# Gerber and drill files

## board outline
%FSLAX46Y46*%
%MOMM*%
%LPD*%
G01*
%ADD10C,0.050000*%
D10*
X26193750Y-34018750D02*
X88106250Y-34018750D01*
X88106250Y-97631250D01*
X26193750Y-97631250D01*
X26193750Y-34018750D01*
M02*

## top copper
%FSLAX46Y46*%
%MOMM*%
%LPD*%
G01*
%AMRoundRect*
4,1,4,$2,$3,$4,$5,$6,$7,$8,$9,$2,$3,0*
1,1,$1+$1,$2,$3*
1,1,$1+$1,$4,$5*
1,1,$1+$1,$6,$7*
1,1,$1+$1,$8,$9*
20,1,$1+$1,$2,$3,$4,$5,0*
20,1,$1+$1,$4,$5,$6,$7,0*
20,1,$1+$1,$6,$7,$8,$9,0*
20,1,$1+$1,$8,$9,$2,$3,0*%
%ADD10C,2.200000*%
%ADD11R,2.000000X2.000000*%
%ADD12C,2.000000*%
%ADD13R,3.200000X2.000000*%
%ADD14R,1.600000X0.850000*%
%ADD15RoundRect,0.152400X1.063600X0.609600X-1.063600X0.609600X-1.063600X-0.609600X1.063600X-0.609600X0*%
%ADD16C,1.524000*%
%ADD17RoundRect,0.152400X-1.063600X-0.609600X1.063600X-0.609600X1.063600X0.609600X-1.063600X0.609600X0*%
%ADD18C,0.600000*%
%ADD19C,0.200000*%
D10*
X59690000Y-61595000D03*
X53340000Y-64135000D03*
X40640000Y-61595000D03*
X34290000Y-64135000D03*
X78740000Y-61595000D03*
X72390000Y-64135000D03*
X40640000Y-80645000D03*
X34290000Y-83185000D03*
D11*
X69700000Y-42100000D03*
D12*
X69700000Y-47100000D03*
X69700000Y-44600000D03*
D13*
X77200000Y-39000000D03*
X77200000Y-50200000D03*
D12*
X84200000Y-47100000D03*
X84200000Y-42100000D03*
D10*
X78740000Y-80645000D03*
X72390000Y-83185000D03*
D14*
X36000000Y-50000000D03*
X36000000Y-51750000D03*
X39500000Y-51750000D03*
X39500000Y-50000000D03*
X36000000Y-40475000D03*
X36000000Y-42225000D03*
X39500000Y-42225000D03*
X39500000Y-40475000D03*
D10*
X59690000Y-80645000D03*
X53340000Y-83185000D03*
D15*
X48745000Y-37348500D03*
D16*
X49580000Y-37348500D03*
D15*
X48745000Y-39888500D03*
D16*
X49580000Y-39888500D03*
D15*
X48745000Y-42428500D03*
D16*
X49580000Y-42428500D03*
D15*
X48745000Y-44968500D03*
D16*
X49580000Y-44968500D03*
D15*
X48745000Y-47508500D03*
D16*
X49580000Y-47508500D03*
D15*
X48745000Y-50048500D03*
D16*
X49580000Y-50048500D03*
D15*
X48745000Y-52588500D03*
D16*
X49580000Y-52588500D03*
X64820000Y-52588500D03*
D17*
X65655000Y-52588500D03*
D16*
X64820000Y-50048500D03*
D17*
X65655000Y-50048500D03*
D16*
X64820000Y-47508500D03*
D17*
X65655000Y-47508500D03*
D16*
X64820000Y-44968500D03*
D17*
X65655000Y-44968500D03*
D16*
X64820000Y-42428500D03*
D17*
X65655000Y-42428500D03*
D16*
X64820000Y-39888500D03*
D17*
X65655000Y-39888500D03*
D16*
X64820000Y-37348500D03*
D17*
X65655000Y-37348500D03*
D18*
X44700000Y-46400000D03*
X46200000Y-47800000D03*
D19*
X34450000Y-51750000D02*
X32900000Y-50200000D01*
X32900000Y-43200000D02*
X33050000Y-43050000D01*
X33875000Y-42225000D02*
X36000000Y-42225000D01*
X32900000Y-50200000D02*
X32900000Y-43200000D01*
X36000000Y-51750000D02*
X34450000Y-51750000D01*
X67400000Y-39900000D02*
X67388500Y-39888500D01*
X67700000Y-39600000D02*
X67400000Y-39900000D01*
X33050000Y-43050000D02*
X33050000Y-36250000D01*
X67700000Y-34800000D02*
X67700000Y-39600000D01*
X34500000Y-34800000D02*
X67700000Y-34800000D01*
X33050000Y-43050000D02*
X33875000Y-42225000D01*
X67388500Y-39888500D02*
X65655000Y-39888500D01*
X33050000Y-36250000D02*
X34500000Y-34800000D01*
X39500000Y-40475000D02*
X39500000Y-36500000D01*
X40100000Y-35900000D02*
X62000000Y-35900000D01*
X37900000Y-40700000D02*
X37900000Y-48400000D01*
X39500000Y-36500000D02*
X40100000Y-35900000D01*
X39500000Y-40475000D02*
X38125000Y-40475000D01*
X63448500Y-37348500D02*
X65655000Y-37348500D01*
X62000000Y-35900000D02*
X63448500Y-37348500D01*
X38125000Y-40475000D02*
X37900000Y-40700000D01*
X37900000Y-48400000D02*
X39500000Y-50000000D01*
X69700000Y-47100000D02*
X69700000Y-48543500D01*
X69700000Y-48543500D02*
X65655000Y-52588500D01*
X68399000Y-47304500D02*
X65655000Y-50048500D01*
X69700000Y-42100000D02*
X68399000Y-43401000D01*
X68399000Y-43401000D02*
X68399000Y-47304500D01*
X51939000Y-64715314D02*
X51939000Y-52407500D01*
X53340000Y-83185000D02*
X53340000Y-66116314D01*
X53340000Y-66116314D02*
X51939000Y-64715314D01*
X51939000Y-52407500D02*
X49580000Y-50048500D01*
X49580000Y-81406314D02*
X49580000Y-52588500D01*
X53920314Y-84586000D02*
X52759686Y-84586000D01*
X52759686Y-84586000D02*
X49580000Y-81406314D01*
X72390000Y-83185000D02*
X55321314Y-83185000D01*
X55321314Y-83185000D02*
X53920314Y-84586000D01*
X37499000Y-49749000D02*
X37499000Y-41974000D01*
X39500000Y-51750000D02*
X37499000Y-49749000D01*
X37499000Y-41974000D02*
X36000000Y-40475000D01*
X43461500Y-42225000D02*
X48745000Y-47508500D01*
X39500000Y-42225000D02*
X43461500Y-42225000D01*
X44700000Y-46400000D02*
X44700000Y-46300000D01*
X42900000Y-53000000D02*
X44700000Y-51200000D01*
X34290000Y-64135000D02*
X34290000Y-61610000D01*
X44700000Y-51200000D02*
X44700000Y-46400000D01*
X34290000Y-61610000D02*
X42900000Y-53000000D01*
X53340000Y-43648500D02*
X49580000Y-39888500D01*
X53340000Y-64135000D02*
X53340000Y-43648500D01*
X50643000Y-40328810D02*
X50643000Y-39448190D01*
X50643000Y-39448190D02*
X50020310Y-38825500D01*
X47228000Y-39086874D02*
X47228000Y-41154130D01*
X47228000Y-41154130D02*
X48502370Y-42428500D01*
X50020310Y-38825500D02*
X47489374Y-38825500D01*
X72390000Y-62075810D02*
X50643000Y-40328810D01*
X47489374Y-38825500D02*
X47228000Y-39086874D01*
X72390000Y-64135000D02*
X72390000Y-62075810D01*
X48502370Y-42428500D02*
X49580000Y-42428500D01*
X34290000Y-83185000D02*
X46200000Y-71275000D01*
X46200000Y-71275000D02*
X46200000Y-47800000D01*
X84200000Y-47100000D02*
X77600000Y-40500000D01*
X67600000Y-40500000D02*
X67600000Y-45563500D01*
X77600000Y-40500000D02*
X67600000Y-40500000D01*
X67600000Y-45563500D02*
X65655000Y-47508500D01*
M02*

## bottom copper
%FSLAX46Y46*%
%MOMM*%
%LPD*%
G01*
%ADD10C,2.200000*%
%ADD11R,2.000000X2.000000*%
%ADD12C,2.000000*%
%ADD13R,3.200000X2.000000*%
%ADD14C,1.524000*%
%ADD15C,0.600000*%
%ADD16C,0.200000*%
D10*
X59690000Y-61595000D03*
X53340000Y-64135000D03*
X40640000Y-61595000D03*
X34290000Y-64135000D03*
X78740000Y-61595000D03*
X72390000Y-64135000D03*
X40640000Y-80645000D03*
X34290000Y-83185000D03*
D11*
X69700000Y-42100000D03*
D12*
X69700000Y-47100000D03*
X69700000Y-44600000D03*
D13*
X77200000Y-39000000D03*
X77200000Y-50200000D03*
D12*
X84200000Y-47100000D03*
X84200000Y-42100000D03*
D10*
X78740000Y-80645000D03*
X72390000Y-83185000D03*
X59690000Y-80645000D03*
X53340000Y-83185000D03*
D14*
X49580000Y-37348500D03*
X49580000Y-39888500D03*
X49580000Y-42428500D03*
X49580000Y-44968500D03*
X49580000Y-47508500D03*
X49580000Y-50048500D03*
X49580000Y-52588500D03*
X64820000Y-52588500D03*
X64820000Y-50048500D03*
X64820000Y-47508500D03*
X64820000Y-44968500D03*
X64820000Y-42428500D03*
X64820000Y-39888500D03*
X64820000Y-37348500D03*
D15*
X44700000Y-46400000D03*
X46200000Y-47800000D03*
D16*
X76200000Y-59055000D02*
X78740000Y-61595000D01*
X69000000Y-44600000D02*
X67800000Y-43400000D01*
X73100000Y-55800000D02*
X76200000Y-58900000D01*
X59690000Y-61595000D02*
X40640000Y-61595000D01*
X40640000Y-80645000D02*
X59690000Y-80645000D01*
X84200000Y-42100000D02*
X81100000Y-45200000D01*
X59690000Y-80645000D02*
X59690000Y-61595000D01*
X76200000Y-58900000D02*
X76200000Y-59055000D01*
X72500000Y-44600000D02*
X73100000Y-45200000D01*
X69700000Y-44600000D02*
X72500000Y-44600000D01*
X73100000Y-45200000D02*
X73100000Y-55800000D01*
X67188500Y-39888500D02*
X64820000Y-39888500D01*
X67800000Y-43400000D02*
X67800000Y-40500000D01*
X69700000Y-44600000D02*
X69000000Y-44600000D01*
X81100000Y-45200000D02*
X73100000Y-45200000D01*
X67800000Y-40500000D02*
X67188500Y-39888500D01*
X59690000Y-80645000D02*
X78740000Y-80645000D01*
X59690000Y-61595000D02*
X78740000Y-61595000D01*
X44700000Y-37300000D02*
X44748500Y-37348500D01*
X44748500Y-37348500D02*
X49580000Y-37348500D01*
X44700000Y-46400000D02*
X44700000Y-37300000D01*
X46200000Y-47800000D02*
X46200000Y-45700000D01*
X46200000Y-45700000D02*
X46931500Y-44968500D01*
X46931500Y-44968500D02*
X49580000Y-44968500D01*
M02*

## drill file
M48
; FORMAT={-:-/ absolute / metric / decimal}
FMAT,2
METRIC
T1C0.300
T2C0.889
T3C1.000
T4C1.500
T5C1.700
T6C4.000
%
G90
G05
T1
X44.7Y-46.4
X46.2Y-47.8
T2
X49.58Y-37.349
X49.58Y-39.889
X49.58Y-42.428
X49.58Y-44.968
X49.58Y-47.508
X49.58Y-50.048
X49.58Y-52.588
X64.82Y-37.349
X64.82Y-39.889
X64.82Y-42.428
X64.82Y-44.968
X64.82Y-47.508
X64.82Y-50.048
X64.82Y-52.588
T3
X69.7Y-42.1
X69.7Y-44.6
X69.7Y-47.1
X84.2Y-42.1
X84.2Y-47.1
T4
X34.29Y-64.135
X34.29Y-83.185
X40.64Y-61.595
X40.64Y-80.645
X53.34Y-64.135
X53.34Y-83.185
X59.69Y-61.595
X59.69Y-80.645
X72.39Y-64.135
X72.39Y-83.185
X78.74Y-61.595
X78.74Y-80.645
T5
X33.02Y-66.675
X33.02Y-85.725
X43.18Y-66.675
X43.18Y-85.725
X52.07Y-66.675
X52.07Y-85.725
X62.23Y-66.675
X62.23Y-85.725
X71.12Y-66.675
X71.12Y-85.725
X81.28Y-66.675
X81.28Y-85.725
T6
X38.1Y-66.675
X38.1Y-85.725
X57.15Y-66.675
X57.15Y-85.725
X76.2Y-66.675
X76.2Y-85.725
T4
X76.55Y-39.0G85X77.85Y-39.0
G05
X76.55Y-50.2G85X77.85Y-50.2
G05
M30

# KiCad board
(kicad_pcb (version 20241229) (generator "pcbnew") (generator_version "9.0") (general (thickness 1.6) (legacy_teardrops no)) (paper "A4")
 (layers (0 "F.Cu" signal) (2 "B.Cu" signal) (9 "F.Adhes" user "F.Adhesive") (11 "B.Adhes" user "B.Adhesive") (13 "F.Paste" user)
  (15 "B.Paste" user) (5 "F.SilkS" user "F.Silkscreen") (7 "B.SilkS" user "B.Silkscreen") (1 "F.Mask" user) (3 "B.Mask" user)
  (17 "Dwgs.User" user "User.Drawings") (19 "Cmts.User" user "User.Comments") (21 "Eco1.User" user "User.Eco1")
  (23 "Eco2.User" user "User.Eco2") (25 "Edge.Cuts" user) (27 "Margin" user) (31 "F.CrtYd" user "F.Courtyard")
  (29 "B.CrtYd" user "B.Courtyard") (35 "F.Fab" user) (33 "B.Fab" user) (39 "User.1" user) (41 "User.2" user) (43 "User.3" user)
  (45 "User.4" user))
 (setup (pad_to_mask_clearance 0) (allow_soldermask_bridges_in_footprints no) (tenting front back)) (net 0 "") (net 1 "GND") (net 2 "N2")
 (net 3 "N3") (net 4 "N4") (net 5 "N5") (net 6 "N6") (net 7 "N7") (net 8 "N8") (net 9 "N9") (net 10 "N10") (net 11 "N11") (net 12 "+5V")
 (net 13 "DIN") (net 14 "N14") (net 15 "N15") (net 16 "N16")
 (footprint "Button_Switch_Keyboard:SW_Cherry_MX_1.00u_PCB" (layer "F.Cu") (at 59.69 61.595)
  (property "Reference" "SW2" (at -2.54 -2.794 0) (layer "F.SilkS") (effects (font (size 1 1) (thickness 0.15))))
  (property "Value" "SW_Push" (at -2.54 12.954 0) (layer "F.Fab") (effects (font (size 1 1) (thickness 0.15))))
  (pad "" np_thru_hole circle (at -7.62 5.08) (size 1.7 1.7) (drill 1.7) (layers "*.Cu" "*.Mask"))
  (pad "" np_thru_hole circle (at -2.54 5.08) (size 4 4) (drill 4) (layers "*.Cu" "*.Mask"))
  (pad "" np_thru_hole circle (at 2.54 5.08) (size 1.7 1.7) (drill 1.7) (layers "*.Cu" "*.Mask"))
  (pad "1" thru_hole circle (at 0 0) (size 2.2 2.2) (drill 1.5) (layers "*.Cu" "*.Mask") (remove_unused_layers no) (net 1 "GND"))
  (pad "2" thru_hole circle (at -6.35 2.54) (size 2.2 2.2) (drill 1.5) (layers "*.Cu" "*.Mask") (remove_unused_layers no) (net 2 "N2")))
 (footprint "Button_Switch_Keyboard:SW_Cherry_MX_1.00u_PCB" (layer "F.Cu") (at 40.64 61.595)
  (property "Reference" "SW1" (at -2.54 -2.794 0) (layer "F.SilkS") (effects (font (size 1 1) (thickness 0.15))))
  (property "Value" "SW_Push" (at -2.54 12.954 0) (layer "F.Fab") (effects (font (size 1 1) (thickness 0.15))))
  (pad "" np_thru_hole circle (at -7.62 5.08) (size 1.7 1.7) (drill 1.7) (layers "*.Cu" "*.Mask"))
  (pad "" np_thru_hole circle (at -2.54 5.08) (size 4 4) (drill 4) (layers "*.Cu" "*.Mask"))
  (pad "" np_thru_hole circle (at 2.54 5.08) (size 1.7 1.7) (drill 1.7) (layers "*.Cu" "*.Mask"))
  (pad "1" thru_hole circle (at 0 0) (size 2.2 2.2) (drill 1.5) (layers "*.Cu" "*.Mask") (remove_unused_layers no) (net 1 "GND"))
  (pad "2" thru_hole circle (at -6.35 2.54) (size 2.2 2.2) (drill 1.5) (layers "*.Cu" "*.Mask") (remove_unused_layers no) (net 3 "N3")))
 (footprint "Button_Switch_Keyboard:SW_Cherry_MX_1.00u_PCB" (layer "F.Cu") (at 78.74 61.595)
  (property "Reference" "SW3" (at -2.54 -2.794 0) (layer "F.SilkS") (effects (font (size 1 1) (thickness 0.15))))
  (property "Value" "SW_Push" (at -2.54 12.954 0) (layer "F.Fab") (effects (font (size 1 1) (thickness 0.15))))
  (pad "" np_thru_hole circle (at -7.62 5.08) (size 1.7 1.7) (drill 1.7) (layers "*.Cu" "*.Mask"))
  (pad "" np_thru_hole circle (at -2.54 5.08) (size 4 4) (drill 4) (layers "*.Cu" "*.Mask"))
  (pad "" np_thru_hole circle (at 2.54 5.08) (size 1.7 1.7) (drill 1.7) (layers "*.Cu" "*.Mask"))
  (pad "1" thru_hole circle (at 0 0) (size 2.2 2.2) (drill 1.5) (layers "*.Cu" "*.Mask") (remove_unused_layers no) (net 1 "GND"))
  (pad "2" thru_hole circle (at -6.35 2.54) (size 2.2 2.2) (drill 1.5) (layers "*.Cu" "*.Mask") (remove_unused_layers no) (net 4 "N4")))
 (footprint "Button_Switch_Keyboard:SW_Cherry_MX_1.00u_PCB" (layer "F.Cu") (at 40.64 80.645)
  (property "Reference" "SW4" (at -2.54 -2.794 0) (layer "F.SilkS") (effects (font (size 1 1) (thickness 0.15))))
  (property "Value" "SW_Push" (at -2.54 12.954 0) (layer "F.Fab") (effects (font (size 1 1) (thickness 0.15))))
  (pad "" np_thru_hole circle (at -7.62 5.08) (size 1.7 1.7) (drill 1.7) (layers "*.Cu" "*.Mask"))
  (pad "" np_thru_hole circle (at -2.54 5.08) (size 4 4) (drill 4) (layers "*.Cu" "*.Mask"))
  (pad "" np_thru_hole circle (at 2.54 5.08) (size 1.7 1.7) (drill 1.7) (layers "*.Cu" "*.Mask"))
  (pad "1" thru_hole circle (at 0 0) (size 2.2 2.2) (drill 1.5) (layers "*.Cu" "*.Mask") (remove_unused_layers no) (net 1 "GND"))
  (pad "2" thru_hole circle (at -6.35 2.54) (size 2.2 2.2) (drill 1.5) (layers "*.Cu" "*.Mask") (remove_unused_layers no) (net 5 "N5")))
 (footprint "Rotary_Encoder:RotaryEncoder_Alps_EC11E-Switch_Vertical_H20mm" (layer "F.Cu") (at 69.7 42.1)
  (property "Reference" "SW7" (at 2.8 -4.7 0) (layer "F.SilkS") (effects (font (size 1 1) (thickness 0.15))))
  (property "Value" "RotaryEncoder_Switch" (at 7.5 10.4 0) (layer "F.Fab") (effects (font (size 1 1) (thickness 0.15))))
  (pad "A" thru_hole rect (at 0 0) (size 2 2) (drill 1) (layers "*.Cu" "*.Mask") (remove_unused_layers no) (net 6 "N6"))
  (pad "B" thru_hole circle (at 0 5) (size 2 2) (drill 1) (layers "*.Cu" "*.Mask") (remove_unused_layers no) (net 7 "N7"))
  (pad "C" thru_hole circle (at 0 2.5) (size 2 2) (drill 1) (layers "*.Cu" "*.Mask") (remove_unused_layers no) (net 1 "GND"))
  (pad "MP" thru_hole rect (at 7.5 -3.1) (size 3.2 2) (drill oval 2.8 1.5) (layers "*.Cu" "*.Mask") (remove_unused_layers no))
  (pad "MP" thru_hole rect (at 7.5 8.1) (size 3.2 2) (drill oval 2.8 1.5) (layers "*.Cu" "*.Mask") (remove_unused_layers no))
  (pad "S1" thru_hole circle (at 14.5 5) (size 2 2) (drill 1) (layers "*.Cu" "*.Mask") (remove_unused_layers no) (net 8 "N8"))
  (pad "S2" thru_hole circle (at 14.5 0) (size 2 2) (drill 1) (layers "*.Cu" "*.Mask") (remove_unused_layers no) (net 1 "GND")))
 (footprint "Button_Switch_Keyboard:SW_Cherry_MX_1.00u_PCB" (layer "F.Cu") (at 78.74 80.645)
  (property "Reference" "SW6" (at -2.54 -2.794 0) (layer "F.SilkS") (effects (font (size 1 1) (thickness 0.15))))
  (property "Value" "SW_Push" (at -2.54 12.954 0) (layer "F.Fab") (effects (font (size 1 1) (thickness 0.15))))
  (pad "" np_thru_hole circle (at -7.62 5.08) (size 1.7 1.7) (drill 1.7) (layers "*.Cu" "*.Mask"))
  (pad "" np_thru_hole circle (at -2.54 5.08) (size 4 4) (drill 4) (layers "*.Cu" "*.Mask"))
  (pad "" np_thru_hole circle (at 2.54 5.08) (size 1.7 1.7) (drill 1.7) (layers "*.Cu" "*.Mask"))
  (pad "1" thru_hole circle (at 0 0) (size 2.2 2.2) (drill 1.5) (layers "*.Cu" "*.Mask") (remove_unused_layers no) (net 1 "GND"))
  (pad "2" thru_hole circle (at -6.35 2.54) (size 2.2 2.2) (drill 1.5) (layers "*.Cu" "*.Mask") (remove_unused_layers no) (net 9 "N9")))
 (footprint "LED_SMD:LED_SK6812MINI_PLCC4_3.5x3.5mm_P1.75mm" (layer "F.Cu") (at 37.75 50.875)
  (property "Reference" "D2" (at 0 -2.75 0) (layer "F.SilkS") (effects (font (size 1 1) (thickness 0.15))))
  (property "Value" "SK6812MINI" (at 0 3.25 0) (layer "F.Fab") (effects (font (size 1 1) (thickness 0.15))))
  (pad "1" smd rect (at -1.75 -0.875) (size 1.6 0.85) (layers "F.Cu" "F.Mask" "F.Paste") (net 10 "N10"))
  (pad "2" smd rect (at -1.75 0.875) (size 1.6 0.85) (layers "F.Cu" "F.Mask" "F.Paste") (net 1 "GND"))
  (pad "3" smd rect (at 1.75 0.875) (size 1.6 0.85) (layers "F.Cu" "F.Mask" "F.Paste") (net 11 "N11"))
  (pad "4" smd rect (at 1.75 -0.875) (size 1.6 0.85) (layers "F.Cu" "F.Mask" "F.Paste") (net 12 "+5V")))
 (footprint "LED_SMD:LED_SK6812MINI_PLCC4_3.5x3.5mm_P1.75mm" (layer "F.Cu") (at 37.75 41.35)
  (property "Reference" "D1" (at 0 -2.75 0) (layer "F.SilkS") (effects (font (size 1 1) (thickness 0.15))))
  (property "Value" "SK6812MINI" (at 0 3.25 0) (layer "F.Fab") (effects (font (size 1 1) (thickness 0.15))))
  (pad "1" smd rect (at -1.75 -0.875) (size 1.6 0.85) (layers "F.Cu" "F.Mask" "F.Paste") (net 11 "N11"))
  (pad "2" smd rect (at -1.75 0.875) (size 1.6 0.85) (layers "F.Cu" "F.Mask" "F.Paste") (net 1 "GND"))
  (pad "3" smd rect (at 1.75 0.875) (size 1.6 0.85) (layers "F.Cu" "F.Mask" "F.Paste") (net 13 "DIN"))
  (pad "4" smd rect (at 1.75 -0.875) (size 1.6 0.85) (layers "F.Cu" "F.Mask" "F.Paste") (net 12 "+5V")))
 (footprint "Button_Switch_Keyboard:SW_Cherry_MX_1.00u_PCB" (layer "F.Cu") (at 59.69 80.645)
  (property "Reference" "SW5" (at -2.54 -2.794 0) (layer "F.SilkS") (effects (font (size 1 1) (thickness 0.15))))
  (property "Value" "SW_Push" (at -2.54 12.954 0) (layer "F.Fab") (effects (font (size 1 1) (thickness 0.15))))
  (pad "" np_thru_hole circle (at -7.62 5.08) (size 1.7 1.7) (drill 1.7) (layers "*.Cu" "*.Mask"))
  (pad "" np_thru_hole circle (at -2.54 5.08) (size 4 4) (drill 4) (layers "*.Cu" "*.Mask"))
  (pad "" np_thru_hole circle (at 2.54 5.08) (size 1.7 1.7) (drill 1.7) (layers "*.Cu" "*.Mask"))
  (pad "1" thru_hole circle (at 0 0) (size 2.2 2.2) (drill 1.5) (layers "*.Cu" "*.Mask") (remove_unused_layers no) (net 1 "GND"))
  (pad "2" thru_hole circle (at -6.35 2.54) (size 2.2 2.2) (drill 1.5) (layers "*.Cu" "*.Mask") (remove_unused_layers no) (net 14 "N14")))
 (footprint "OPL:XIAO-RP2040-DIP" (layer "F.Cu") (at 57.2 44.9685)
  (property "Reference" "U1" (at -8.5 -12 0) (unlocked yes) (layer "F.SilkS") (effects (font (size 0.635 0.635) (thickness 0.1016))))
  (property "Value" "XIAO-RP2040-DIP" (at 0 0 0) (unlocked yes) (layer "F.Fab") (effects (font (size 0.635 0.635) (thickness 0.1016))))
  (pad "1" smd roundrect (at -8.455 -7.62 180) (size 2.432 1.524) (layers "F.Cu" "F.Mask") (roundrect_rratio 0.1) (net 3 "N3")
   (thermal_bridge_angle 45))
  (pad "1" thru_hole circle (at -7.62 -7.62 180) (size 1.524 1.524) (drill 0.889) (layers "*.Cu" "*.Mask") (remove_unused_layers no)
   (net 3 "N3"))
  (pad "2" smd roundrect (at -8.455 -5.08 180) (size 2.432 1.524) (layers "F.Cu" "F.Mask") (roundrect_rratio 0.1) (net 2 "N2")
   (thermal_bridge_angle 45))
  (pad "2" thru_hole circle (at -7.62 -5.08 180) (size 1.524 1.524) (drill 0.889) (layers "*.Cu" "*.Mask") (remove_unused_layers no)
   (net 2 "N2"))
  (pad "3" smd roundrect (at -8.455 -2.54 180) (size 2.432 1.524) (layers "F.Cu" "F.Mask") (roundrect_rratio 0.1) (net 4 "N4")
   (thermal_bridge_angle 45))
  (pad "3" thru_hole circle (at -7.62 -2.54 180) (size 1.524 1.524) (drill 0.889) (layers "*.Cu" "*.Mask") (remove_unused_layers no)
   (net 4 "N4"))
  (pad "4" smd roundrect (at -8.455 0 180) (size 2.432 1.524) (layers "F.Cu" "F.Mask") (roundrect_rratio 0.1) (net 5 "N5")
   (thermal_bridge_angle 45))
  (pad "4" thru_hole circle (at -7.62 0 180) (size 1.524 1.524) (drill 0.889) (layers "*.Cu" "*.Mask") (remove_unused_layers no)
   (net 5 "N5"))
  (pad "5" smd roundrect (at -8.455 2.54 180) (size 2.432 1.524) (layers "F.Cu" "F.Mask") (roundrect_rratio 0.1) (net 13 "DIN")
   (thermal_bridge_angle 45))
  (pad "5" thru_hole circle (at -7.62 2.54 180) (size 1.524 1.524) (drill 0.889) (layers "*.Cu" "*.Mask") (remove_unused_layers no)
   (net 13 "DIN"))
  (pad "6" smd roundrect (at -8.455 5.08 180) (size 2.432 1.524) (layers "F.Cu" "F.Mask") (roundrect_rratio 0.1) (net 14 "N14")
   (thermal_bridge_angle 45))
  (pad "6" thru_hole circle (at -7.62 5.08 180) (size 1.524 1.524) (drill 0.889) (layers "*.Cu" "*.Mask") (remove_unused_layers no)
   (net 14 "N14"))
  (pad "7" smd roundrect (at -8.455 7.62 180) (size 2.432 1.524) (layers "F.Cu" "F.Mask") (roundrect_rratio 0.1) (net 9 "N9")
   (thermal_bridge_angle 45))
  (pad "7" thru_hole circle (at -7.62 7.62 180) (size 1.524 1.524) (drill 0.889) (layers "*.Cu" "*.Mask") (remove_unused_layers no)
   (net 9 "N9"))
  (pad "8" thru_hole circle (at 7.62 7.62) (size 1.524 1.524) (drill 0.889) (layers "*.Cu" "*.Mask") (remove_unused_layers no) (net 7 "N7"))
  (pad "8" smd roundrect (at 8.455 7.62) (size 2.432 1.524) (layers "F.Cu" "F.Mask") (roundrect_rratio 0.1) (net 7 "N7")
   (thermal_bridge_angle 45))
  (pad "9" thru_hole circle (at 7.62 5.08) (size 1.524 1.524) (drill 0.889) (layers "*.Cu" "*.Mask") (remove_unused_layers no) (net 6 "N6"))
  (pad "9" smd roundrect (at 8.455 5.08) (size 2.432 1.524) (layers "F.Cu" "F.Mask") (roundrect_rratio 0.1) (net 6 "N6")
   (thermal_bridge_angle 45))
  (pad "10" thru_hole circle (at 7.62 2.54) (size 1.524 1.524) (drill 0.889) (layers "*.Cu" "*.Mask") (remove_unused_layers no) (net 8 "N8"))
  (pad "10" smd roundrect (at 8.455 2.54) (size 2.432 1.524) (layers "F.Cu" "F.Mask") (roundrect_rratio 0.1) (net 8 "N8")
   (thermal_bridge_angle 45))
  (pad "11" thru_hole circle (at 7.62 0) (size 1.524 1.524) (drill 0.889) (layers "*.Cu" "*.Mask") (remove_unused_layers no) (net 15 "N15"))
  (pad "11" smd roundrect (at 8.455 0) (size 2.432 1.524) (layers "F.Cu" "F.Mask") (roundrect_rratio 0.1) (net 15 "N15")
   (thermal_bridge_angle 45))
  (pad "12" thru_hole circle (at 7.62 -2.54) (size 1.524 1.524) (drill 0.889) (layers "*.Cu" "*.Mask") (remove_unused_layers no)
   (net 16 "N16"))
  (pad "12" smd roundrect (at 8.455 -2.54) (size 2.432 1.524) (layers "F.Cu" "F.Mask") (roundrect_rratio 0.1) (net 16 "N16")
   (thermal_bridge_angle 45))
  (pad "13" thru_hole circle (at 7.62 -5.08) (size 1.524 1.524) (drill 0.889) (layers "*.Cu" "*.Mask") (remove_unused_layers no)
   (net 1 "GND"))
  (pad "13" smd roundrect (at 8.455 -5.08) (size 2.432 1.524) (layers "F.Cu" "F.Mask") (roundrect_rratio 0.1) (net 1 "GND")
   (thermal_bridge_angle 45))
  (pad "14" thru_hole circle (at 7.62 -7.62) (size 1.524 1.524) (drill 0.889) (layers "*.Cu" "*.Mask") (remove_unused_layers no)
   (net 12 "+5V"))
  (pad "14" smd roundrect (at 8.455 -7.62) (size 2.432 1.524) (layers "F.Cu" "F.Mask") (roundrect_rratio 0.1) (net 12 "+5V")
   (thermal_bridge_angle 45)))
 (gr_rect (start 26.19375 34.01875) (end 88.10625 97.63125) (stroke (width 0.05) (type default)) (fill no) (layer "Edge.Cuts"))
 (segment (start 34.45 51.75) (end 32.9 50.2) (width 0.2) (layer "F.Cu") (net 1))
 (segment (start 32.9 43.2) (end 33.05 43.05) (width 0.2) (layer "F.Cu") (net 1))
 (segment (start 33.875 42.225) (end 36 42.225) (width 0.2) (layer "F.Cu") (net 1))
 (segment (start 32.9 50.2) (end 32.9 43.2) (width 0.2) (layer "F.Cu") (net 1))
 (segment (start 36 51.75) (end 34.45 51.75) (width 0.2) (layer "F.Cu") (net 1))
 (segment (start 67.4 39.9) (end 67.3885 39.8885) (width 0.2) (layer "F.Cu") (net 1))
 (segment (start 67.7 39.6) (end 67.4 39.9) (width 0.2) (layer "F.Cu") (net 1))
 (segment (start 33.05 43.05) (end 33.05 36.25) (width 0.2) (layer "F.Cu") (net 1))
 (segment (start 67.7 34.8) (end 67.7 39.6) (width 0.2) (layer "F.Cu") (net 1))
 (segment (start 34.5 34.8) (end 67.7 34.8) (width 0.2) (layer "F.Cu") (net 1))
 (segment (start 33.05 43.05) (end 33.875 42.225) (width 0.2) (layer "F.Cu") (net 1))
 (segment (start 67.3885 39.8885) (end 65.655 39.8885) (width 0.2) (layer "F.Cu") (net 1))
 (segment (start 33.05 36.25) (end 34.5 34.8) (width 0.2) (layer "F.Cu") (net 1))
 (segment (start 76.2 59.055) (end 78.74 61.595) (width 0.2) (layer "B.Cu") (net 1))
 (segment (start 69 44.6) (end 67.8 43.4) (width 0.2) (layer "B.Cu") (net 1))
 (segment (start 73.1 55.8) (end 76.2 58.9) (width 0.2) (layer "B.Cu") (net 1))
 (segment (start 59.69 61.595) (end 40.64 61.595) (width 0.2) (layer "B.Cu") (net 1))
 (segment (start 40.64 80.645) (end 59.69 80.645) (width 0.2) (layer "B.Cu") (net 1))
 (segment (start 84.2 42.1) (end 81.1 45.2) (width 0.2) (layer "B.Cu") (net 1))
 (segment (start 59.69 80.645) (end 59.69 61.595) (width 0.2) (layer "B.Cu") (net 1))
 (segment (start 76.2 58.9) (end 76.2 59.055) (width 0.2) (layer "B.Cu") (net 1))
 (segment (start 72.5 44.6) (end 73.1 45.2) (width 0.2) (layer "B.Cu") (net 1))
 (segment (start 69.7 44.6) (end 72.5 44.6) (width 0.2) (layer "B.Cu") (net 1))
 (segment (start 73.1 45.2) (end 73.1 55.8) (width 0.2) (layer "B.Cu") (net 1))
 (segment (start 67.1885 39.8885) (end 64.82 39.8885) (width 0.2) (layer "B.Cu") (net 1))
 (segment (start 67.8 43.4) (end 67.8 40.5) (width 0.2) (layer "B.Cu") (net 1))
 (segment (start 69.7 44.6) (end 69 44.6) (width 0.2) (layer "B.Cu") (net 1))
 (segment (start 81.1 45.2) (end 73.1 45.2) (width 0.2) (layer "B.Cu") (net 1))
 (segment (start 67.8 40.5) (end 67.1885 39.8885) (width 0.2) (layer "B.Cu") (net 1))
 (segment (start 59.69 80.645) (end 78.74 80.645) (width 0.2) (layer "B.Cu") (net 1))
 (segment (start 59.69 61.595) (end 78.74 61.595) (width 0.2) (layer "B.Cu") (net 1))
 (segment (start 39.5 40.475) (end 39.5 36.5) (width 0.2) (layer "F.Cu") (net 12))
 (segment (start 40.1 35.9) (end 62 35.9) (width 0.2) (layer "F.Cu") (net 12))
 (segment (start 37.9 40.7) (end 37.9 48.4) (width 0.2) (layer "F.Cu") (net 12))
 (segment (start 39.5 36.5) (end 40.1 35.9) (width 0.2) (layer "F.Cu") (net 12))
 (segment (start 39.5 40.475) (end 38.125 40.475) (width 0.2) (layer "F.Cu") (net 12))
 (segment (start 63.4485 37.3485) (end 65.655 37.3485) (width 0.2) (layer "F.Cu") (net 12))
 (segment (start 62 35.9) (end 63.4485 37.3485) (width 0.2) (layer "F.Cu") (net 12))
 (segment (start 38.125 40.475) (end 37.9 40.7) (width 0.2) (layer "F.Cu") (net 12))
 (segment (start 37.9 48.4) (end 39.5 50) (width 0.2) (layer "F.Cu") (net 12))
 (segment (start 69.7 47.1) (end 69.7 48.5435) (width 0.2) (layer "F.Cu") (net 7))
 (segment (start 69.7 48.5435) (end 65.655 52.5885) (width 0.2) (layer "F.Cu") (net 7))
 (segment (start 68.399 47.3045) (end 65.655 50.0485) (width 0.2) (layer "F.Cu") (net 6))
 (segment (start 69.7 42.1) (end 68.399 43.401) (width 0.2) (layer "F.Cu") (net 6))
 (segment (start 68.399 43.401) (end 68.399 47.3045) (width 0.2) (layer "F.Cu") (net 6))
 (segment (start 51.939 64.715314) (end 51.939 52.4075) (width 0.2) (layer "F.Cu") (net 14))
 (segment (start 53.34 83.185) (end 53.34 66.116314) (width 0.2) (layer "F.Cu") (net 14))
 (segment (start 53.34 66.116314) (end 51.939 64.715314) (width 0.2) (layer "F.Cu") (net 14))
 (segment (start 51.939 52.4075) (end 49.58 50.0485) (width 0.2) (layer "F.Cu") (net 14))
 (segment (start 49.58 81.406314) (end 49.58 52.5885) (width 0.2) (layer "F.Cu") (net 9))
 (segment (start 53.920314 84.586) (end 52.759686 84.586) (width 0.2) (layer "F.Cu") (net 9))
 (segment (start 52.759686 84.586) (end 49.58 81.406314) (width 0.2) (layer "F.Cu") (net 9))
 (segment (start 72.39 83.185) (end 55.321314 83.185) (width 0.2) (layer "F.Cu") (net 9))
 (segment (start 55.321314 83.185) (end 53.920314 84.586) (width 0.2) (layer "F.Cu") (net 9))
 (segment (start 37.499 49.749) (end 37.499 41.974) (width 0.2) (layer "F.Cu") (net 11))
 (segment (start 39.5 51.75) (end 37.499 49.749) (width 0.2) (layer "F.Cu") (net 11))
 (segment (start 37.499 41.974) (end 36 40.475) (width 0.2) (layer "F.Cu") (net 11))
 (segment (start 43.4615 42.225) (end 48.745 47.5085) (width 0.2) (layer "F.Cu") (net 13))
 (segment (start 39.5 42.225) (end 43.4615 42.225) (width 0.2) (layer "F.Cu") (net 13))
 (segment (start 44.7 46.4) (end 44.7 46.3) (width 0.2) (layer "F.Cu") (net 3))
 (segment (start 42.9 53) (end 44.7 51.2) (width 0.2) (layer "F.Cu") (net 3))
 (segment (start 34.29 64.135) (end 34.29 61.61) (width 0.2) (layer "F.Cu") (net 3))
 (segment (start 44.7 51.2) (end 44.7 46.4) (width 0.2) (layer "F.Cu") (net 3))
 (segment (start 34.29 61.61) (end 42.9 53) (width 0.2) (layer "F.Cu") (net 3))
 (via (at 44.7 46.4) (size 0.6) (drill 0.3) (layers "F.Cu" "B.Cu") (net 3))
 (segment (start 44.7 37.3) (end 44.7485 37.3485) (width 0.2) (layer "B.Cu") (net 3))
 (segment (start 44.7485 37.3485) (end 49.58 37.3485) (width 0.2) (layer "B.Cu") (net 3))
 (segment (start 44.7 46.4) (end 44.7 37.3) (width 0.2) (layer "B.Cu") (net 3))
 (segment (start 53.34 43.6485) (end 49.58 39.8885) (width 0.2) (layer "F.Cu") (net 2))
 (segment (start 53.34 64.135) (end 53.34 43.6485) (width 0.2) (layer "F.Cu") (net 2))
 (segment (start 50.643 40.32881) (end 50.643 39.44819) (width 0.2) (layer "F.Cu") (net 4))
 (segment (start 50.643 39.44819) (end 50.02031 38.8255) (width 0.2) (layer "F.Cu") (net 4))
 (segment (start 47.228 39.086874) (end 47.228 41.15413) (width 0.2) (layer "F.Cu") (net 4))
 (segment (start 47.228 41.15413) (end 48.50237 42.4285) (width 0.2) (layer "F.Cu") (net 4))
 (segment (start 50.02031 38.8255) (end 47.489374 38.8255) (width 0.2) (layer "F.Cu") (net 4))
 (segment (start 72.39 62.07581) (end 50.643 40.32881) (width 0.2) (layer "F.Cu") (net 4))
 (segment (start 47.489374 38.8255) (end 47.228 39.086874) (width 0.2) (layer "F.Cu") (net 4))
 (segment (start 72.39 64.135) (end 72.39 62.07581) (width 0.2) (layer "F.Cu") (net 4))
 (segment (start 48.50237 42.4285) (end 49.58 42.4285) (width 0.2) (layer "F.Cu") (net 4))
 (segment (start 34.29 83.185) (end 46.2 71.275) (width 0.2) (layer "F.Cu") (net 5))
 (segment (start 46.2 71.275) (end 46.2 47.8) (width 0.2) (layer "F.Cu") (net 5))
 (via (at 46.2 47.8) (size 0.6) (drill 0.3) (layers "F.Cu" "B.Cu") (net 5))
 (segment (start 46.2 47.8) (end 46.2 45.7) (width 0.2) (layer "B.Cu") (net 5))
 (segment (start 46.2 45.7) (end 46.9315 44.9685) (width 0.2) (layer "B.Cu") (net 5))
 (segment (start 46.9315 44.9685) (end 49.58 44.9685) (width 0.2) (layer "B.Cu") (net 5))
 (segment (start 84.2 47.1) (end 77.6 40.5) (width 0.2) (layer "F.Cu") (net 8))
 (segment (start 67.6 40.5) (end 67.6 45.5635) (width 0.2) (layer "F.Cu") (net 8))
 (segment (start 77.6 40.5) (end 67.6 40.5) (width 0.2) (layer "F.Cu") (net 8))
 (segment (start 67.6 45.5635) (end 65.655 47.5085) (width 0.2) (layer "F.Cu") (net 8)))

